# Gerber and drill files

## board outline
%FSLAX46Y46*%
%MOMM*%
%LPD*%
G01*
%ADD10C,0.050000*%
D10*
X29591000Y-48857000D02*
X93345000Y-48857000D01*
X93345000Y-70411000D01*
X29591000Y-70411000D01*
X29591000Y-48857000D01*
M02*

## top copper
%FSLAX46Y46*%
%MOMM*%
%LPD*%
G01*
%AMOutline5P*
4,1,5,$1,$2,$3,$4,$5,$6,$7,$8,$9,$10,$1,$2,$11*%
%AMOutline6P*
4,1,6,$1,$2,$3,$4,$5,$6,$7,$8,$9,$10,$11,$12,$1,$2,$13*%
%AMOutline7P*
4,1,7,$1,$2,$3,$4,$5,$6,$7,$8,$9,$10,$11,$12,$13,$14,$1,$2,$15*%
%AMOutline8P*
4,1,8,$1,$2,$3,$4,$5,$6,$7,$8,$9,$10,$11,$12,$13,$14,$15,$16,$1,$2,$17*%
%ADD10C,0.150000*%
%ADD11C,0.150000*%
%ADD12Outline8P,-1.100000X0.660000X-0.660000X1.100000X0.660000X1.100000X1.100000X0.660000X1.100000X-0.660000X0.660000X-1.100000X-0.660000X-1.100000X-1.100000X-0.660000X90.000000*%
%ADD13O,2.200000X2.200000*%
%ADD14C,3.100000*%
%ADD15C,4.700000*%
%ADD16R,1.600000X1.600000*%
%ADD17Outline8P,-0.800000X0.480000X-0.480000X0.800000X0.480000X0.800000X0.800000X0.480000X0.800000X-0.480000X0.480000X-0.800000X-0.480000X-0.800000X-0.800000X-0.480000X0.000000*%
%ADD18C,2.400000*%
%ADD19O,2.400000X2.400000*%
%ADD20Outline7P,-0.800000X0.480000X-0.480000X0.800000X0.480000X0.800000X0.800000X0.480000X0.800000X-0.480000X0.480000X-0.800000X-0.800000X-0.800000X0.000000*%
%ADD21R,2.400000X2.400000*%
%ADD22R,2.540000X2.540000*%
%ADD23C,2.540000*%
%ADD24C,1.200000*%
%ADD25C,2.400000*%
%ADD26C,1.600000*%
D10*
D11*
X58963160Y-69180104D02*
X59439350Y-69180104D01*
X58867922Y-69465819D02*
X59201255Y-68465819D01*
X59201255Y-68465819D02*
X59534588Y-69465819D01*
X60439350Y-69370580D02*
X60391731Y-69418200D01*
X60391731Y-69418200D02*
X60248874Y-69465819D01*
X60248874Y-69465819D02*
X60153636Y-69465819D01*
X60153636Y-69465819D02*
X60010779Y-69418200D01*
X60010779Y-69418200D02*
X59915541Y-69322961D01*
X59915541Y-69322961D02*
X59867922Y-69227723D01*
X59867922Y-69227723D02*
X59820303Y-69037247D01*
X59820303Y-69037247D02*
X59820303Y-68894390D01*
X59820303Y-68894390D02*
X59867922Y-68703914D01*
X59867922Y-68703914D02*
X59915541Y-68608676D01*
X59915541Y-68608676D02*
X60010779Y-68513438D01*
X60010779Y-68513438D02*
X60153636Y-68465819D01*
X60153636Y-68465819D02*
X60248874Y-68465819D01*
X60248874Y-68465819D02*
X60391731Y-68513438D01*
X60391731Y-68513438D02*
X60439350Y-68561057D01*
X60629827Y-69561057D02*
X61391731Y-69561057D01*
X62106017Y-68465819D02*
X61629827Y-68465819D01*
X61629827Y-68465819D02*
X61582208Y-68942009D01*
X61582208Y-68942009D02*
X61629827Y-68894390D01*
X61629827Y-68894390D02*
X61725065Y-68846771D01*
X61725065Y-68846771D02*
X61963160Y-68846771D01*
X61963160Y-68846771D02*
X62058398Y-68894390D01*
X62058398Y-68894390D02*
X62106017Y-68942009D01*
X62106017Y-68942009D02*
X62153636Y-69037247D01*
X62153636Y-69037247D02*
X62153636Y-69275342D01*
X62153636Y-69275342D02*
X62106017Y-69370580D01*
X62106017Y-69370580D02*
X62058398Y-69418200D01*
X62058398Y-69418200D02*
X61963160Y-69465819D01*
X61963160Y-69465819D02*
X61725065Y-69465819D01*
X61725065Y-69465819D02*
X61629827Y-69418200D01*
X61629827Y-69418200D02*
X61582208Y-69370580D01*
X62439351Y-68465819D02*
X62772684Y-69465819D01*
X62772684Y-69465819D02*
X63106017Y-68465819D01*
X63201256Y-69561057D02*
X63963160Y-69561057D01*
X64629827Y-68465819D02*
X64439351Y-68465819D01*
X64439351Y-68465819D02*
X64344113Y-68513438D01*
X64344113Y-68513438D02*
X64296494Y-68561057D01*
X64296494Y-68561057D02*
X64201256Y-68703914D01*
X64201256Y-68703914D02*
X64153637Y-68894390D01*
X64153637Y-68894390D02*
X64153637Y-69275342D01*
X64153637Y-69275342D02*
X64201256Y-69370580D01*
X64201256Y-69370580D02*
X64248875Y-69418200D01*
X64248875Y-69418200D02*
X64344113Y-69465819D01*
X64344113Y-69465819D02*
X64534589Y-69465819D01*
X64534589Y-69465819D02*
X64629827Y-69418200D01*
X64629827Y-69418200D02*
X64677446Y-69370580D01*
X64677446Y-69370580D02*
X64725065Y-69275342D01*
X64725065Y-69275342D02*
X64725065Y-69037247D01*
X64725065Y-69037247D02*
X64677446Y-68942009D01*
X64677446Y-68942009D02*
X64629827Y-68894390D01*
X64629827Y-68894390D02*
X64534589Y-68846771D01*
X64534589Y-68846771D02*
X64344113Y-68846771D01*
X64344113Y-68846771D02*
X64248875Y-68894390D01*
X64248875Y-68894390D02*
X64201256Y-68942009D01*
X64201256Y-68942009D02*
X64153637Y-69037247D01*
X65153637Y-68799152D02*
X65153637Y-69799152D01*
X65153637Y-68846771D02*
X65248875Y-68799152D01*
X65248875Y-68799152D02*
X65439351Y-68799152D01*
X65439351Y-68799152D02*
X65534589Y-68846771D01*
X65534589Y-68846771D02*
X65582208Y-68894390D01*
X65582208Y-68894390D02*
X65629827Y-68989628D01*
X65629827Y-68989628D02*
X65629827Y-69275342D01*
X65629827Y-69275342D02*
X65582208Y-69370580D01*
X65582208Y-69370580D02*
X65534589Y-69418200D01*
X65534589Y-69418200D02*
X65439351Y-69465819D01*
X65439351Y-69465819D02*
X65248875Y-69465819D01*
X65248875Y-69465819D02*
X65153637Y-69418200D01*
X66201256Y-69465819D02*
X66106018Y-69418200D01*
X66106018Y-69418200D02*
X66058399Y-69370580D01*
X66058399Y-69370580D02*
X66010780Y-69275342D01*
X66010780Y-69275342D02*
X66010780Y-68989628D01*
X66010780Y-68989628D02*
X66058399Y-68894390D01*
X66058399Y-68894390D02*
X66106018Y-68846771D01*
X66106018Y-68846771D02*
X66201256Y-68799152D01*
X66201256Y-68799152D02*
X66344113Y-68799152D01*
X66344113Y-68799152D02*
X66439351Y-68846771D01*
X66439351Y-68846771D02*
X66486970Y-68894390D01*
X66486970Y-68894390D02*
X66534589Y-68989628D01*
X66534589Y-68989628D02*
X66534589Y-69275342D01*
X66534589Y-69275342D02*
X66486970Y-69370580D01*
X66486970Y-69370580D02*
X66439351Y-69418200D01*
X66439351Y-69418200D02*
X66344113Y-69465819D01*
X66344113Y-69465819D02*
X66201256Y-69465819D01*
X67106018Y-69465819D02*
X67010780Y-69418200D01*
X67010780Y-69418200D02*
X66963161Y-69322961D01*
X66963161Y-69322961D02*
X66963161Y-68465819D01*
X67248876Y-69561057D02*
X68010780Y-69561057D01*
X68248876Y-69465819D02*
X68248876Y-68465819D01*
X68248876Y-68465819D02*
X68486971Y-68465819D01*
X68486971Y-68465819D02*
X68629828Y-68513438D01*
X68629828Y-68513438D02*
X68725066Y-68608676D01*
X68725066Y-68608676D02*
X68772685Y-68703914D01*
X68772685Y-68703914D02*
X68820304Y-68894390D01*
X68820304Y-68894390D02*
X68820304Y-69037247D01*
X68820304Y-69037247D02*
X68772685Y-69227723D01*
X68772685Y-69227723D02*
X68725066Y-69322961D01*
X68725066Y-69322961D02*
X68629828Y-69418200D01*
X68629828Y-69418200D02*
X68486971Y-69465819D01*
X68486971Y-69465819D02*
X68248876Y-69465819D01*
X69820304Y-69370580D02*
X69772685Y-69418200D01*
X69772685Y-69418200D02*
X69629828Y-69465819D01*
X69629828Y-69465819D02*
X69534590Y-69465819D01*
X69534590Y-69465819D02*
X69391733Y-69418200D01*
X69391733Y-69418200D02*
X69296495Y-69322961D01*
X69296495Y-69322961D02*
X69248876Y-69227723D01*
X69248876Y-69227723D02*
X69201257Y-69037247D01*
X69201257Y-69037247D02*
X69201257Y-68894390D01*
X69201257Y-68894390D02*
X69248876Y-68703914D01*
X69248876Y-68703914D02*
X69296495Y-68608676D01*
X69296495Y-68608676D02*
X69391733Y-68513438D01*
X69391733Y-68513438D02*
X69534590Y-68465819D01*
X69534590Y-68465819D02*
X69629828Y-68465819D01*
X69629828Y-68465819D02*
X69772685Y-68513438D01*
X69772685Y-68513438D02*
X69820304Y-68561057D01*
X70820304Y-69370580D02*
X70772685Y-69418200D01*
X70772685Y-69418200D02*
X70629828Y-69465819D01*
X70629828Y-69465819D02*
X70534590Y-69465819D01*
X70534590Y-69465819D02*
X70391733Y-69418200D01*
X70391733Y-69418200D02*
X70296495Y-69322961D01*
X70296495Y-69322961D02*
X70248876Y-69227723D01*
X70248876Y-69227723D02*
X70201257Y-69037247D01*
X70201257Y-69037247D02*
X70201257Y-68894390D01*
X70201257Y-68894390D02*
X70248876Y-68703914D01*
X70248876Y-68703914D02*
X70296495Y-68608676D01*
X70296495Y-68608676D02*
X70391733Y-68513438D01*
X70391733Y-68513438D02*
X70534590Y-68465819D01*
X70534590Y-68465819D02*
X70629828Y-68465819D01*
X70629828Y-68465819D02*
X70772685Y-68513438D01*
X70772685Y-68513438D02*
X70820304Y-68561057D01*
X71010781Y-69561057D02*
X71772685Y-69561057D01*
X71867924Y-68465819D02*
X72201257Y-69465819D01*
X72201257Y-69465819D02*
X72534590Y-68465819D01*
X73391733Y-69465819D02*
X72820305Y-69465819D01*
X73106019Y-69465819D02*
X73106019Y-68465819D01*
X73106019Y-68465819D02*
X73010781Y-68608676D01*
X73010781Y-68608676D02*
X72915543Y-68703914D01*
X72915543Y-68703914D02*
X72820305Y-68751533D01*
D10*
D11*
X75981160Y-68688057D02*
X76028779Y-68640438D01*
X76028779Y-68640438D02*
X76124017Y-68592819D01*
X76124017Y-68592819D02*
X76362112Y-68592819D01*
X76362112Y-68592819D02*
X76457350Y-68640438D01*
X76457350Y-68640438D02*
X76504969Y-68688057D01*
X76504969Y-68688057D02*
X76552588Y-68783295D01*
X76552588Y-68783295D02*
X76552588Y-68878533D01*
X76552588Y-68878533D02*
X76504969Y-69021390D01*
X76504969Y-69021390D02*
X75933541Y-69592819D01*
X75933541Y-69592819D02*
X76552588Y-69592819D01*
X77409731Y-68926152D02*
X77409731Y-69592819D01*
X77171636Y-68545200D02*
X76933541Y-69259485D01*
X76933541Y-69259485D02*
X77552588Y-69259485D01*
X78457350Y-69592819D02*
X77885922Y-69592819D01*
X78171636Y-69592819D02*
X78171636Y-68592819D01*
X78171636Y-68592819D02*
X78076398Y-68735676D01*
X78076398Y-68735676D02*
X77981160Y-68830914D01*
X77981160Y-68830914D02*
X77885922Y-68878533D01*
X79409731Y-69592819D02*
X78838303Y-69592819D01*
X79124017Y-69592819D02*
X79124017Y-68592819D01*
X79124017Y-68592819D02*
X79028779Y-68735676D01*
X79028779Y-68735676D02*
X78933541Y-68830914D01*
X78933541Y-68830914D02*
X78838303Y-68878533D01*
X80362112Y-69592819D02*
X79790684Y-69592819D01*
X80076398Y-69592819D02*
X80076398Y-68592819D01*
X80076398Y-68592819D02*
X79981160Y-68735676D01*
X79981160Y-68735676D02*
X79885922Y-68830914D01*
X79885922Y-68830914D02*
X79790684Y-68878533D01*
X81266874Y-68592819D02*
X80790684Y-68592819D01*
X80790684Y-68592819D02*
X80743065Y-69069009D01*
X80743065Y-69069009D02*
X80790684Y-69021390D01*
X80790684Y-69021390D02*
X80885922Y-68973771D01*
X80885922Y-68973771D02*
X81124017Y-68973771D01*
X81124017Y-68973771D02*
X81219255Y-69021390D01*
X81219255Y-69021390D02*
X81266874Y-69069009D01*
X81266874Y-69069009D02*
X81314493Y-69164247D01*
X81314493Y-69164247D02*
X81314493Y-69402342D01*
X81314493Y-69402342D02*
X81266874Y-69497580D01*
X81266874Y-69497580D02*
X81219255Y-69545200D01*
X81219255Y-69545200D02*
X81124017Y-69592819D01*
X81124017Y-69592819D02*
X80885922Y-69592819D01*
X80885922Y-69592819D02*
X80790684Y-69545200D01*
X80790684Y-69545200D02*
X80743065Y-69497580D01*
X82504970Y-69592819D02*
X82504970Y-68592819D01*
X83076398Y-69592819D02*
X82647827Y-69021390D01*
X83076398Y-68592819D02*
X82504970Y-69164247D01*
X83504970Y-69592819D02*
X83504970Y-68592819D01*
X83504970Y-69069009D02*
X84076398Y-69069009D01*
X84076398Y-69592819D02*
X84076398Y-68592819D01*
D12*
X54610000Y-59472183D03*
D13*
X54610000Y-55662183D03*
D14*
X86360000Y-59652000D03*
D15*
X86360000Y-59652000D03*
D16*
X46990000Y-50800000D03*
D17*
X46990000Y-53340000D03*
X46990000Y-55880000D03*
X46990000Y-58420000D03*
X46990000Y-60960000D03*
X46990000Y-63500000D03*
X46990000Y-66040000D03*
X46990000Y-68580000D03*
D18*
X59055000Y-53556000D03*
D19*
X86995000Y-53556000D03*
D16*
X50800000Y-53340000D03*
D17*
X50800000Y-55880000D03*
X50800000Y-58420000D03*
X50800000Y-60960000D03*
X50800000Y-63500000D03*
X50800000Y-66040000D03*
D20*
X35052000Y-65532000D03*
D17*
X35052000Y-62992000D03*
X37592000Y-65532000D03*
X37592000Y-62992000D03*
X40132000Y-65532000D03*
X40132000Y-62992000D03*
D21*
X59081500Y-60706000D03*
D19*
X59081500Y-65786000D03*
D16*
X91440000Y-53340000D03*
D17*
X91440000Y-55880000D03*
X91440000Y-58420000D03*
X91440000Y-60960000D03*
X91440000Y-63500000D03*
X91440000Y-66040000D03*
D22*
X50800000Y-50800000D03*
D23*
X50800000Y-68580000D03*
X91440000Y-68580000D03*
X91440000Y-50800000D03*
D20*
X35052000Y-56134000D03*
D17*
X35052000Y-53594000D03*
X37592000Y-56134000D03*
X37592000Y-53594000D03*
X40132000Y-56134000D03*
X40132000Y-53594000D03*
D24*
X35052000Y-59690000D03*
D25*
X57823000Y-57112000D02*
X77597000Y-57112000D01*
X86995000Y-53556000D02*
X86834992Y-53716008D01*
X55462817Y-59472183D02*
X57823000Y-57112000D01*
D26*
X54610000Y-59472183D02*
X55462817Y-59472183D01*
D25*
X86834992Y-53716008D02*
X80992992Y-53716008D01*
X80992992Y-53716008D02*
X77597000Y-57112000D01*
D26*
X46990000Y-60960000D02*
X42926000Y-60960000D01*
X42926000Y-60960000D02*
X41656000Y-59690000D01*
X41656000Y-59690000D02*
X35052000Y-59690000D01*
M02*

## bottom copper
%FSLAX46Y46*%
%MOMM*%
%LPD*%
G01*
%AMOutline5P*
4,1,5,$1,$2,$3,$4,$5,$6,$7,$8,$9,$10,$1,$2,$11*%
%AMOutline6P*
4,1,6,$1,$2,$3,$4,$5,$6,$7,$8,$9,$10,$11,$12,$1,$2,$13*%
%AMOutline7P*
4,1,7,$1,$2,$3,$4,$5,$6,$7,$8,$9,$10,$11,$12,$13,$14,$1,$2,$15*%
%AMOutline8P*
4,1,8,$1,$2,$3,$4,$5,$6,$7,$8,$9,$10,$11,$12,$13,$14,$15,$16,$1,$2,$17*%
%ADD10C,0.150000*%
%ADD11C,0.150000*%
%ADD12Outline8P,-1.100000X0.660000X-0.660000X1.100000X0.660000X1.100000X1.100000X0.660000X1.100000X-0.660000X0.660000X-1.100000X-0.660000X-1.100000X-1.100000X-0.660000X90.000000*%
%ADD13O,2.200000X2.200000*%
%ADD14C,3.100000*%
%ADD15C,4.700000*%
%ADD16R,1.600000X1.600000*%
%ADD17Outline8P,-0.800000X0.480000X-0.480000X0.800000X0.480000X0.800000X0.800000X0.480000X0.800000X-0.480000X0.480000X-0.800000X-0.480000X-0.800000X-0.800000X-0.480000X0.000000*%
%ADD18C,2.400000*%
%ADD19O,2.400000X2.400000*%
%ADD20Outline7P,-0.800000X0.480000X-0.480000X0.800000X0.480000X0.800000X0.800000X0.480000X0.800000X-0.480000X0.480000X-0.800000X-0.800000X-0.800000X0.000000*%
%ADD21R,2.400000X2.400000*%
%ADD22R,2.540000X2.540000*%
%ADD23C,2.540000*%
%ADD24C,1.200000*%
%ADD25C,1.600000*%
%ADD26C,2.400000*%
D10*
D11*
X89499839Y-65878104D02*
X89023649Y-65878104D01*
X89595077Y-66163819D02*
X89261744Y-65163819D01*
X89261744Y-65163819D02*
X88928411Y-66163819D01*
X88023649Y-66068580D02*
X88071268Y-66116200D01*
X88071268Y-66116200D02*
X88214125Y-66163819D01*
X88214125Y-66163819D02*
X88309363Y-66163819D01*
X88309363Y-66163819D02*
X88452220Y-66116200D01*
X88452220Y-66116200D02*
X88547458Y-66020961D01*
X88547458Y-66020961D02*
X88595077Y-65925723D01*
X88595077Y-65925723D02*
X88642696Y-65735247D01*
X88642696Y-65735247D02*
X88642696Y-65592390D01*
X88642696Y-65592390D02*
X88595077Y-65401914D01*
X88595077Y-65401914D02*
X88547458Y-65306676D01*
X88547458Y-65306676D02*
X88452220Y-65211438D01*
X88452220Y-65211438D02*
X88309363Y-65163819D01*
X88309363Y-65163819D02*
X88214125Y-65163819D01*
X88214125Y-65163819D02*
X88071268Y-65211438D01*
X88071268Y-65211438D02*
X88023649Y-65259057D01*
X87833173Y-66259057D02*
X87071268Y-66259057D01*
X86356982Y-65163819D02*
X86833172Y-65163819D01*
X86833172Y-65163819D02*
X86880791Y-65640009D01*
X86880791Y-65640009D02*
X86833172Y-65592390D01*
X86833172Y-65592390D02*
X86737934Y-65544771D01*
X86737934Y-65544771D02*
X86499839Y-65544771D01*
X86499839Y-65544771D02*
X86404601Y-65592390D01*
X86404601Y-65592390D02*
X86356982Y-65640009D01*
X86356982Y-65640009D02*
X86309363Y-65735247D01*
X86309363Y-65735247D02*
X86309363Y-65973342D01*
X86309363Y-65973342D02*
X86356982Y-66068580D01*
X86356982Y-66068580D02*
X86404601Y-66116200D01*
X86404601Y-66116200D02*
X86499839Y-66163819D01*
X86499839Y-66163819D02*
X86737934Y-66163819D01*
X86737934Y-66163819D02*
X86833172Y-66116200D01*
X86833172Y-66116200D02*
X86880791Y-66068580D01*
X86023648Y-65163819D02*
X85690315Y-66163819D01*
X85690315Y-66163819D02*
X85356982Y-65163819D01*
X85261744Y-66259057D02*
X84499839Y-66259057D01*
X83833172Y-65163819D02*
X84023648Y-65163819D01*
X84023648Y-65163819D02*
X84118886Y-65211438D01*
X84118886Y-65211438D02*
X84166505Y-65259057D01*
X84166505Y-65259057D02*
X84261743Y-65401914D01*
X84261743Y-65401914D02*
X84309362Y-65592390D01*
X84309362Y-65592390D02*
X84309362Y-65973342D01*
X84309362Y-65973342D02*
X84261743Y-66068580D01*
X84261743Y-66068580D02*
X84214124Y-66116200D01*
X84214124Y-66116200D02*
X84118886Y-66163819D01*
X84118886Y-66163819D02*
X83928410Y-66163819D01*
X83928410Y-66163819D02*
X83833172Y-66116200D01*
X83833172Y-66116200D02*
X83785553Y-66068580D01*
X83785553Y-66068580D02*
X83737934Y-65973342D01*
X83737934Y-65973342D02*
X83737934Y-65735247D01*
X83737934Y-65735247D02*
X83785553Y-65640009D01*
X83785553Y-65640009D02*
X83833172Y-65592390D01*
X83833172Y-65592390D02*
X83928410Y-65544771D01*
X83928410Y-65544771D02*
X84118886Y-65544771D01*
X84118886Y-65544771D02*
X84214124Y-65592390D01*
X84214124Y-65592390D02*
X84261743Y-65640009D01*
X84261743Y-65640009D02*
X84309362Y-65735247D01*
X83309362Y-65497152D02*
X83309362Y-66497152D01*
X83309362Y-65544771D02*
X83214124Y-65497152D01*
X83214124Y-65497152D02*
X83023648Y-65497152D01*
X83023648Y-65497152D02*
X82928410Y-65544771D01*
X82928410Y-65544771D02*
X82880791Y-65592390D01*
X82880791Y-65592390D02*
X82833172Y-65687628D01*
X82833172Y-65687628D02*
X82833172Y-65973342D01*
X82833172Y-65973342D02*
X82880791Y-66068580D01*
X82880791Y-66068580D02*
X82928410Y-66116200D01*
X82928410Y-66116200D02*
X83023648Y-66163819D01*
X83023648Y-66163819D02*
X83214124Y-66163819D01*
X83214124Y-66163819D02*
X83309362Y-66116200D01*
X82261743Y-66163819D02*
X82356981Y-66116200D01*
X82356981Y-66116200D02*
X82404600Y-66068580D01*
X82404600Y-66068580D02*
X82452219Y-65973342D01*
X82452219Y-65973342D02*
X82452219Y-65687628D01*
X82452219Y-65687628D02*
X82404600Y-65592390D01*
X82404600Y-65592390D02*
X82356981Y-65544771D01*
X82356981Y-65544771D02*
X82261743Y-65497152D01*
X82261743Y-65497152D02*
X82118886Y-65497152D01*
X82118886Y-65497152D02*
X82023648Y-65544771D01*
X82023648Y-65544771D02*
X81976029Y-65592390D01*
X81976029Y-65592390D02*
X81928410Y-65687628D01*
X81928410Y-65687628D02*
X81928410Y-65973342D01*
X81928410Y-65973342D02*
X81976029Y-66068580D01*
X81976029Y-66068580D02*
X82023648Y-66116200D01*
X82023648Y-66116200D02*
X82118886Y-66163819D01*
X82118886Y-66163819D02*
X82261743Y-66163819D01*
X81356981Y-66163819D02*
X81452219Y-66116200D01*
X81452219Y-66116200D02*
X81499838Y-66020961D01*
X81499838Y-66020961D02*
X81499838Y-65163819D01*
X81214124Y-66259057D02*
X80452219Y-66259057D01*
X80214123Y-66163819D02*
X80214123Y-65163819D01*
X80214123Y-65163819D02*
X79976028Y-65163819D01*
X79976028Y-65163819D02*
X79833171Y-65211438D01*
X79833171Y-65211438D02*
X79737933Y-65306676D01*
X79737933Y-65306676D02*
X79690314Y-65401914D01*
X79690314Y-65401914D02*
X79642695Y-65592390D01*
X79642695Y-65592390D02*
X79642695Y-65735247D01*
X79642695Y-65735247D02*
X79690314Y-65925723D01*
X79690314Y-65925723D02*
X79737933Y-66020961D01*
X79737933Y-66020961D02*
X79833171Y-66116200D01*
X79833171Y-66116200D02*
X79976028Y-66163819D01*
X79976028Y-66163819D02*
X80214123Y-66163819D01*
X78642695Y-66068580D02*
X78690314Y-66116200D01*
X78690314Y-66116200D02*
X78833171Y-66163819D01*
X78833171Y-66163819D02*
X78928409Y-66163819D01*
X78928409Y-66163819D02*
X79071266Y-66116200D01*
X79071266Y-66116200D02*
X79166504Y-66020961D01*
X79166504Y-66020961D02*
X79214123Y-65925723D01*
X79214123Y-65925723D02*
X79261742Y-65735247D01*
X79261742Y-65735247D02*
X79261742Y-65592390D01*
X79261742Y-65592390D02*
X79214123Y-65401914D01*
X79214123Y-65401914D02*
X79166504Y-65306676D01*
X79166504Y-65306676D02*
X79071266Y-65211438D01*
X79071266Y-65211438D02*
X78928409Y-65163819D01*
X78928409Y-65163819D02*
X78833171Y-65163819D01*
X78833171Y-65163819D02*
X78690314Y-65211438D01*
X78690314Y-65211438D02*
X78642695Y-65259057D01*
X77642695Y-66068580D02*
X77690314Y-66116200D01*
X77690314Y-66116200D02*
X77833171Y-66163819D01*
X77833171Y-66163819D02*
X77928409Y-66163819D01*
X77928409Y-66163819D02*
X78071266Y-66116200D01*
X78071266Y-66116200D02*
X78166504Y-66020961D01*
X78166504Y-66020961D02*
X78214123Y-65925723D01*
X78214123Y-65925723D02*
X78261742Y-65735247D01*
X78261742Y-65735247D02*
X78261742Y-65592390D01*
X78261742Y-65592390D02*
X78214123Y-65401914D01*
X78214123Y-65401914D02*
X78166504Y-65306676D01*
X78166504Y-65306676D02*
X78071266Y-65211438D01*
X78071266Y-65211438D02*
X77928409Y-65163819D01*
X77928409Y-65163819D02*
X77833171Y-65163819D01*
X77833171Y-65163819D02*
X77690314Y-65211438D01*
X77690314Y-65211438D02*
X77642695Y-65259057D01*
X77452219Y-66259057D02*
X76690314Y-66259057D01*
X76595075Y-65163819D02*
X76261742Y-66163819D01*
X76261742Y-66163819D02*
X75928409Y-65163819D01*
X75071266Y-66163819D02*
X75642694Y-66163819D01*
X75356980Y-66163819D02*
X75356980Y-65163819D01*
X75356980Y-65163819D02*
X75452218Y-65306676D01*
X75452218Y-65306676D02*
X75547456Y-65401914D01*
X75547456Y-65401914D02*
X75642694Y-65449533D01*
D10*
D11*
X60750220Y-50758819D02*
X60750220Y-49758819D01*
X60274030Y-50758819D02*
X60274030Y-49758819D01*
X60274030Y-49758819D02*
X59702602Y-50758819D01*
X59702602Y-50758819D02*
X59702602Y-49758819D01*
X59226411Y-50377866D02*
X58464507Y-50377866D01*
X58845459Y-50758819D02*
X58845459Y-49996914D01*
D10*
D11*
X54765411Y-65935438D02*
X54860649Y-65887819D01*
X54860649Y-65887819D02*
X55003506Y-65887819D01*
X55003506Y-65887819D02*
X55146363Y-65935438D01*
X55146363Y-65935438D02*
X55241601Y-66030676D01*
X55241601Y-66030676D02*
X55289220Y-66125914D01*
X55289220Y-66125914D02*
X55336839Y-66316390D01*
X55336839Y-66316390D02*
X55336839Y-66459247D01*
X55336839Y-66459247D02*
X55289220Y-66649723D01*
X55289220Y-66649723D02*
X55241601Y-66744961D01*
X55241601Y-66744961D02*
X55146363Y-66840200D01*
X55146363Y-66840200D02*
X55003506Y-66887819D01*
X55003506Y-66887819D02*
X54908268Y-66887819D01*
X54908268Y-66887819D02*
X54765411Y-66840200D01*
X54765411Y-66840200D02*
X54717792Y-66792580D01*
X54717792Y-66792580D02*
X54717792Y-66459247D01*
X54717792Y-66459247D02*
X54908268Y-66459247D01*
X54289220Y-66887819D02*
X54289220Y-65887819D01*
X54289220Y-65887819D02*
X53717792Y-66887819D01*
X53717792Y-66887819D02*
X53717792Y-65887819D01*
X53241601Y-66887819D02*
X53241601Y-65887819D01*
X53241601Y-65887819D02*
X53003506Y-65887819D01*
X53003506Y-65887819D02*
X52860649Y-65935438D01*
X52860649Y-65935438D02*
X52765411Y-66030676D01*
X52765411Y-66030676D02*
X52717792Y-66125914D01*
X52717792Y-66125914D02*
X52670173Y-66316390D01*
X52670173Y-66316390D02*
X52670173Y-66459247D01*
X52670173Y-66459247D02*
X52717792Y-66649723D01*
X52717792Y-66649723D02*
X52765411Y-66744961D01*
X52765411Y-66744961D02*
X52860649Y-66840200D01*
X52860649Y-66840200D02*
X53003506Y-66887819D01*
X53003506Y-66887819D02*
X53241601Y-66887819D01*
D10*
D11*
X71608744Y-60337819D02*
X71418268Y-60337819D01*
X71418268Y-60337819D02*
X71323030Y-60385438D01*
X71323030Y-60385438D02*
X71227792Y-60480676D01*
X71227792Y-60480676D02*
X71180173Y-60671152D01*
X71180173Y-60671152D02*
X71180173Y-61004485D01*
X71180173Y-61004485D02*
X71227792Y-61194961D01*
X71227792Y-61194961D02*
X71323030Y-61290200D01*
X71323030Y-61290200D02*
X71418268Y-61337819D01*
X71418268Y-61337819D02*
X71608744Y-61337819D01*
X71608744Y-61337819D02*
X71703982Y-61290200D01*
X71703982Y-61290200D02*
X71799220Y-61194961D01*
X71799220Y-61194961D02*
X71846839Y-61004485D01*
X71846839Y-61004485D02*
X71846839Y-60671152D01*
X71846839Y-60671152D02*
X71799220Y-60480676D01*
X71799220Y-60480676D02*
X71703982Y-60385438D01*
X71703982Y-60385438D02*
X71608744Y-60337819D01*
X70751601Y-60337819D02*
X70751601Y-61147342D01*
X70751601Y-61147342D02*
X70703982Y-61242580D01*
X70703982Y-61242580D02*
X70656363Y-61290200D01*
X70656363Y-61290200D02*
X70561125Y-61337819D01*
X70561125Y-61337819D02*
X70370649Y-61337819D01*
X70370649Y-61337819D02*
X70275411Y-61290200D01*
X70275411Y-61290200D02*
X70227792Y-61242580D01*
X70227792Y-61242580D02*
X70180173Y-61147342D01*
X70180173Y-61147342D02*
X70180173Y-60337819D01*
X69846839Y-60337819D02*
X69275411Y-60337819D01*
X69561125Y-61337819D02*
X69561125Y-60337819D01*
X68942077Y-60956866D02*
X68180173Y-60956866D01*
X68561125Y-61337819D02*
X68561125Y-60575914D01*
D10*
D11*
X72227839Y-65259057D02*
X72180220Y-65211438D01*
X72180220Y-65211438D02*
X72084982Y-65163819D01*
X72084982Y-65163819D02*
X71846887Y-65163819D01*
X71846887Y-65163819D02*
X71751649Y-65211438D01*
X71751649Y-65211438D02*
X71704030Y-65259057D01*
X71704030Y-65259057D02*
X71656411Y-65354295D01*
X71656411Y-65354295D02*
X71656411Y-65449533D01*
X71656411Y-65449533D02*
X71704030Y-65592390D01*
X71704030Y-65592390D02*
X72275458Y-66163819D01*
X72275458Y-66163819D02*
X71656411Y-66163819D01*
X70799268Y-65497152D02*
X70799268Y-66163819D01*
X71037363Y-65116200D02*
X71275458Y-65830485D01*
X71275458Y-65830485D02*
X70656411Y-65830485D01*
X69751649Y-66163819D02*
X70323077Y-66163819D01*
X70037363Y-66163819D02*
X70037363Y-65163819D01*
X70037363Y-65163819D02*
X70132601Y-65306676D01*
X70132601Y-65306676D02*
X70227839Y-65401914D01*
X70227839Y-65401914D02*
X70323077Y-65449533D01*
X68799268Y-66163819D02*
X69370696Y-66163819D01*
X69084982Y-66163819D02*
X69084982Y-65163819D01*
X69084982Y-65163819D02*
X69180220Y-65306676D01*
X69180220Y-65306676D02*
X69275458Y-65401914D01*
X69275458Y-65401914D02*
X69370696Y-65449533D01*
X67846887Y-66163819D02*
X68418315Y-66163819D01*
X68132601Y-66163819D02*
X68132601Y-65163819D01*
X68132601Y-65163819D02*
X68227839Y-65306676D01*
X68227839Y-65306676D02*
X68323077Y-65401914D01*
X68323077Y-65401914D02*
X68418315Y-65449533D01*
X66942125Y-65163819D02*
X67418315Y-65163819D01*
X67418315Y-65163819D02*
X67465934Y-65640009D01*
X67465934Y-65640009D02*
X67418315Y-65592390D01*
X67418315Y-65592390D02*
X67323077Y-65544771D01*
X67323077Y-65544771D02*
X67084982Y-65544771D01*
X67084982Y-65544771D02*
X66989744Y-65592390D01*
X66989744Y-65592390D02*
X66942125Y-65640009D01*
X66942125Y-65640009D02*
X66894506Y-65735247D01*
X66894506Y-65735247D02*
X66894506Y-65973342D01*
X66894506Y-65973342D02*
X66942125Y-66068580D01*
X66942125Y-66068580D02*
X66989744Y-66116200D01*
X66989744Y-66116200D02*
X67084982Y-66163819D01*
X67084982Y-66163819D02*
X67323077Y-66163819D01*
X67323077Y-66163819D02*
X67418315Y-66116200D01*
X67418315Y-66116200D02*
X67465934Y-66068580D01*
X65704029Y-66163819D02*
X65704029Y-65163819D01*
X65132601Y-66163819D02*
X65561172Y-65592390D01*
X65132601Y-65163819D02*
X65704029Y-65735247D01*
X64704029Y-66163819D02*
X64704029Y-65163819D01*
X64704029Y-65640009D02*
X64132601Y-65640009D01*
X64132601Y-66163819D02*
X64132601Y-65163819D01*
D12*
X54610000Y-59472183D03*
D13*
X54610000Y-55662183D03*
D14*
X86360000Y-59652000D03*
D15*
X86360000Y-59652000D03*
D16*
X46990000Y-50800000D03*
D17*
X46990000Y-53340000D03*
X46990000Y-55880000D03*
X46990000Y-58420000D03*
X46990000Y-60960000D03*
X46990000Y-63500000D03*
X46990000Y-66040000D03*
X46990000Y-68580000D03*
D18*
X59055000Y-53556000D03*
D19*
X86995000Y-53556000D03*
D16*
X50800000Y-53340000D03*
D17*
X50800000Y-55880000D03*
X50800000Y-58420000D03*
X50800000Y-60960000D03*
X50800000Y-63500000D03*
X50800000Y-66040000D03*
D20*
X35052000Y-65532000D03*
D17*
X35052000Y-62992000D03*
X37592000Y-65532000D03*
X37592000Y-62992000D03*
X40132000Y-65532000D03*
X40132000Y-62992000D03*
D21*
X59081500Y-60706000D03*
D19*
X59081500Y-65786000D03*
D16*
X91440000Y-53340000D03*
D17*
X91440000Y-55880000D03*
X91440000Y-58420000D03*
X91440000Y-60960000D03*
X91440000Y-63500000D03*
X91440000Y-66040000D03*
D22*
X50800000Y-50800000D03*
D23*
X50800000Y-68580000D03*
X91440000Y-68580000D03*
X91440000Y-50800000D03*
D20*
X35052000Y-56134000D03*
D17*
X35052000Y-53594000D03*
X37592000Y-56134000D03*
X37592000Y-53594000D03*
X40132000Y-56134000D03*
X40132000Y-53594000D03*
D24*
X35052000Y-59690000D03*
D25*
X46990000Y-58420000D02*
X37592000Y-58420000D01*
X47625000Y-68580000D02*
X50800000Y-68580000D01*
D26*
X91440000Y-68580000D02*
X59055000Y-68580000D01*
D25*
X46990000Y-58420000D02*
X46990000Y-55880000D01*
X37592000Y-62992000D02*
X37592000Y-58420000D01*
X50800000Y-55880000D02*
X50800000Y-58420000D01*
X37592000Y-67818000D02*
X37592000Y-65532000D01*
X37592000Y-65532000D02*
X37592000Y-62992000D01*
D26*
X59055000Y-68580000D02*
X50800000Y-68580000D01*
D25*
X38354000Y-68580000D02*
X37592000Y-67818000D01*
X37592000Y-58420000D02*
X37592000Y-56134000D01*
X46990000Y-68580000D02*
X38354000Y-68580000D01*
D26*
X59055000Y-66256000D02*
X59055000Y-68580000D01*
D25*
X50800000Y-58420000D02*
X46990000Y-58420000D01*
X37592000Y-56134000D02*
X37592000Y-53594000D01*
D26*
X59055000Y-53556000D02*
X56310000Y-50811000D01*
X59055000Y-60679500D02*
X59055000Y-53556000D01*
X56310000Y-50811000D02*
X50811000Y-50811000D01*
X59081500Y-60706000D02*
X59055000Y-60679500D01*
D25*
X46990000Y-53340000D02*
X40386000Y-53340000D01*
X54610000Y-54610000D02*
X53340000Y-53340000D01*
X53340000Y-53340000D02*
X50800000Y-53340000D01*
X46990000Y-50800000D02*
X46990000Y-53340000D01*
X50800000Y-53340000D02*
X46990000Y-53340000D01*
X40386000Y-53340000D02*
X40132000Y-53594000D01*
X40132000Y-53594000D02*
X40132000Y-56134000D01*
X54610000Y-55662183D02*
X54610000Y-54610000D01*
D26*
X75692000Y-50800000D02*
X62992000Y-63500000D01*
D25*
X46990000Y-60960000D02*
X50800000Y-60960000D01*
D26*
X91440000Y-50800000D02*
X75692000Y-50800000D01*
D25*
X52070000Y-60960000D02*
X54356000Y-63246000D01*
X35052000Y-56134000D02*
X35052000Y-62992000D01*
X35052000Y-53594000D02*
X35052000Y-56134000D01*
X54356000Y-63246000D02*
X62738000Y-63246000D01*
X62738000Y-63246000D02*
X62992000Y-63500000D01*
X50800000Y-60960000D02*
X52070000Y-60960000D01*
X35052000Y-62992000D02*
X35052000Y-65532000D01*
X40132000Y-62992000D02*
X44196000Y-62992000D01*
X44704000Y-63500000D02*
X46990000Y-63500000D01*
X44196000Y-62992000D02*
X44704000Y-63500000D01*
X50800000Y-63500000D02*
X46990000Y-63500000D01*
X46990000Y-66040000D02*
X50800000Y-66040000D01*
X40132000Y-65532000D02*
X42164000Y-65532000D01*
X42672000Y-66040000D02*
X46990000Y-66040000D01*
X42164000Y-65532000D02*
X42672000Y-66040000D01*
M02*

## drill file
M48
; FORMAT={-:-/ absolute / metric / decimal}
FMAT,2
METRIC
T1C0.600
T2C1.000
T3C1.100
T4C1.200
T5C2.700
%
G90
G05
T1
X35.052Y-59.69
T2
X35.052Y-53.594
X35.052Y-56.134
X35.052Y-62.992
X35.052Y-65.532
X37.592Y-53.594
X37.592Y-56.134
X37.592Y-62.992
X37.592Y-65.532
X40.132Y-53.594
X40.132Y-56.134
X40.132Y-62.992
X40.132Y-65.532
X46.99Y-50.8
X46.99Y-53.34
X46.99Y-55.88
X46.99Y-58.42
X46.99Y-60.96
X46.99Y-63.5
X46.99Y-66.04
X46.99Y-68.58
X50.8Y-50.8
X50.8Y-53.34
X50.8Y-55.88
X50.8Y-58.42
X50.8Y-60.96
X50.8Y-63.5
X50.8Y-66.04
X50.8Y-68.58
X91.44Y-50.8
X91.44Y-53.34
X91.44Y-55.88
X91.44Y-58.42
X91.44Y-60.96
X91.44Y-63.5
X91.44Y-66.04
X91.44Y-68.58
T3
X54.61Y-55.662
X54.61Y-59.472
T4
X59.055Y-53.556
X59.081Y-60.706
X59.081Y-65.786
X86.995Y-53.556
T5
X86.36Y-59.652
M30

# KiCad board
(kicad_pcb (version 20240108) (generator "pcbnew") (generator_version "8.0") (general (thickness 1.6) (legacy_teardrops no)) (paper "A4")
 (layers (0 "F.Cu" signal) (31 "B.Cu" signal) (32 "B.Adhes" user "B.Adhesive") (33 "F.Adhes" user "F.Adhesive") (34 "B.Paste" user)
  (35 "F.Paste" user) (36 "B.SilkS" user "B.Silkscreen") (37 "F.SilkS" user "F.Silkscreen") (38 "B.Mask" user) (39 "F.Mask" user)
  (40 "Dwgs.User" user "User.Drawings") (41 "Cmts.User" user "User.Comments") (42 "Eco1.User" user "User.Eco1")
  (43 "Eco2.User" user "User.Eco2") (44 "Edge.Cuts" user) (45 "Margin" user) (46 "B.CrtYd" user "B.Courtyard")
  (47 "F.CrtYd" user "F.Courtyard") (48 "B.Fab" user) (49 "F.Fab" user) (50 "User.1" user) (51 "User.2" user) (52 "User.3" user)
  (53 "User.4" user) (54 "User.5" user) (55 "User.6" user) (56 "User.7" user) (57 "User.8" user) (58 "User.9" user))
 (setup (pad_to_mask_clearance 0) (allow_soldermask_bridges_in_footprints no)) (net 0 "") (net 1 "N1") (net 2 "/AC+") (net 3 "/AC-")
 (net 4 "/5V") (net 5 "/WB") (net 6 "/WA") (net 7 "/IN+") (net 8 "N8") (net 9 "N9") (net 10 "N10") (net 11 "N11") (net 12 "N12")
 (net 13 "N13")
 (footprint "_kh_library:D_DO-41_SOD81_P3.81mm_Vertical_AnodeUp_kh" (layer "F.Cu") (at 54.61 59.472183 90)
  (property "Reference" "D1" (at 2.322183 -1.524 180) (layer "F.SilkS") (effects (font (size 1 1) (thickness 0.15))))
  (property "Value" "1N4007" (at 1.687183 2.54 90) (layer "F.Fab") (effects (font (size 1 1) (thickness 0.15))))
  (pad "1" thru_hole roundrect (at 0 0 90) (size 2.2 2.2) (drill 1.1) (layers "*.Cu" "*.Mask") (remove_unused_layers no)
   (roundrect_rratio 0) (chamfer_ratio 0.2) (chamfer top_left top_right bottom_left bottom_right) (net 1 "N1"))
  (pad "2" thru_hole oval (at 3.81 0 90) (size 2.2 2.2) (drill 1.1) (layers "*.Cu" "*.Mask") (remove_unused_layers no) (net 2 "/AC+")))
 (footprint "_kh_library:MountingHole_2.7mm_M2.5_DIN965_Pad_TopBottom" (layer "F.Cu") (at 86.36 59.652)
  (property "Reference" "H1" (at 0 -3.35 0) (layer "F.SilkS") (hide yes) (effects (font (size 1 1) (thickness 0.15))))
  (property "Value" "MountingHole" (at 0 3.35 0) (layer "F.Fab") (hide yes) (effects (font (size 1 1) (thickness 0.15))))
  (pad "1" thru_hole circle (at 0 0) (size 3.1 3.1) (drill 2.7) (layers "*.Cu" "*.Mask") (remove_unused_layers no))
  (pad "1" connect circle (at 0 0) (size 4.7 4.7) (layers "F.Cu" "F.Mask"))
  (pad "1" connect circle (at 0 0) (size 4.7 4.7) (layers "B.Cu" "B.Mask")))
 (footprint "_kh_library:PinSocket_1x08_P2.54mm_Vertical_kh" (layer "F.Cu") (at 46.99 50.8)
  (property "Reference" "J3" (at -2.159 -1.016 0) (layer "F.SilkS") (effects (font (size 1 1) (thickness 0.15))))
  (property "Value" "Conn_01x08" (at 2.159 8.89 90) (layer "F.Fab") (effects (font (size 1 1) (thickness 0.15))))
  (pad "1" thru_hole rect (at 0 0) (size 1.6 1.6) (drill 1) (layers "*.Cu" "*.Mask") (remove_unused_layers no) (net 2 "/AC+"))
  (pad "2" thru_hole roundrect (at 0 2.54) (size 1.6 1.6) (drill 1) (layers "*.Cu" "*.Mask") (remove_unused_layers no) (roundrect_rratio 0)
   (chamfer_ratio 0.2) (chamfer top_left top_right bottom_left bottom_right) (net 2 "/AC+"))
  (pad "3" thru_hole roundrect (at 0 5.08) (size 1.6 1.6) (drill 1) (layers "*.Cu" "*.Mask") (remove_unused_layers no) (roundrect_rratio 0)
   (chamfer_ratio 0.2) (chamfer top_left top_right bottom_left bottom_right) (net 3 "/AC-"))
  (pad "4" thru_hole roundrect (at 0 7.62) (size 1.6 1.6) (drill 1) (layers "*.Cu" "*.Mask") (remove_unused_layers no) (roundrect_rratio 0)
   (chamfer_ratio 0.2) (chamfer top_left top_right bottom_left bottom_right) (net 3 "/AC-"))
  (pad "5" thru_hole roundrect (at 0 10.16) (size 1.6 1.6) (drill 1) (layers "*.Cu" "*.Mask") (remove_unused_layers no) (roundrect_rratio 0)
   (chamfer_ratio 0.2) (chamfer top_left top_right bottom_left bottom_right) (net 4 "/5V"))
  (pad "6" thru_hole roundrect (at 0 12.7) (size 1.6 1.6) (drill 1) (layers "*.Cu" "*.Mask") (remove_unused_layers no) (roundrect_rratio 0)
   (chamfer_ratio 0.2) (chamfer top_left top_right bottom_left bottom_right) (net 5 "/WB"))
  (pad "7" thru_hole roundrect (at 0 15.24) (size 1.6 1.6) (drill 1) (layers "*.Cu" "*.Mask") (remove_unused_layers no) (roundrect_rratio 0)
   (chamfer_ratio 0.2) (chamfer top_left top_right bottom_left bottom_right) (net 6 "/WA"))
  (pad "8" thru_hole roundrect (at 0 17.78) (size 1.6 1.6) (drill 1) (layers "*.Cu" "*.Mask") (remove_unused_layers no) (roundrect_rratio 0)
   (chamfer_ratio 0.2) (chamfer top_left top_right bottom_left bottom_right) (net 3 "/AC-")))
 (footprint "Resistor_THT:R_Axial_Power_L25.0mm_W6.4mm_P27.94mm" (layer "F.Cu") (at 59.055 53.556)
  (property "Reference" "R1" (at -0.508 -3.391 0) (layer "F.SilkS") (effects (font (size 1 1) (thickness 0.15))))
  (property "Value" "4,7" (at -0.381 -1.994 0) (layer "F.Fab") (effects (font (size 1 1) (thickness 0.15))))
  (pad "1" thru_hole circle (at 0 0) (size 2.4 2.4) (drill 1.2) (layers "*.Cu" "*.Mask") (remove_unused_layers no) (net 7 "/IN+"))
  (pad "2" thru_hole oval (at 27.94 0) (size 2.4 2.4) (drill 1.2) (layers "*.Cu" "*.Mask") (remove_unused_layers no) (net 1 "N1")))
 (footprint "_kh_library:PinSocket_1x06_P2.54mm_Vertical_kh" (layer "F.Cu") (at 50.8 53.34)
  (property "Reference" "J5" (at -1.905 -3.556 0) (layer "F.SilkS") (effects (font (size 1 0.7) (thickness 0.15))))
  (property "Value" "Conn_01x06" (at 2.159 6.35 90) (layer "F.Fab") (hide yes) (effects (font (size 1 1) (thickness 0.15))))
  (pad "1" thru_hole rect (at 0 0) (size 1.6 1.6) (drill 1) (layers "*.Cu" "*.Mask") (remove_unused_layers no) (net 2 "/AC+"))
  (pad "2" thru_hole roundrect (at 0 2.54) (size 1.6 1.6) (drill 1) (layers "*.Cu" "*.Mask") (remove_unused_layers no) (roundrect_rratio 0)
   (chamfer_ratio 0.2) (chamfer top_left top_right bottom_left bottom_right) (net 3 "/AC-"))
  (pad "3" thru_hole roundrect (at 0 5.08) (size 1.6 1.6) (drill 1) (layers "*.Cu" "*.Mask") (remove_unused_layers no) (roundrect_rratio 0)
   (chamfer_ratio 0.2) (chamfer top_left top_right bottom_left bottom_right) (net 3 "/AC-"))
  (pad "4" thru_hole roundrect (at 0 7.62) (size 1.6 1.6) (drill 1) (layers "*.Cu" "*.Mask") (remove_unused_layers no) (roundrect_rratio 0)
   (chamfer_ratio 0.2) (chamfer top_left top_right bottom_left bottom_right) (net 4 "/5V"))
  (pad "5" thru_hole roundrect (at 0 10.16) (size 1.6 1.6) (drill 1) (layers "*.Cu" "*.Mask") (remove_unused_layers no) (roundrect_rratio 0)
   (chamfer_ratio 0.2) (chamfer top_left top_right bottom_left bottom_right) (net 5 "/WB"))
  (pad "6" thru_hole roundrect (at 0 12.7) (size 1.6 1.6) (drill 1) (layers "*.Cu" "*.Mask") (remove_unused_layers no) (roundrect_rratio 0)
   (chamfer_ratio 0.2) (chamfer top_left top_right bottom_left bottom_right) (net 6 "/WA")))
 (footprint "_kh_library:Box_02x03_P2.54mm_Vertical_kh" (layer "F.Cu") (at 35.052 65.532)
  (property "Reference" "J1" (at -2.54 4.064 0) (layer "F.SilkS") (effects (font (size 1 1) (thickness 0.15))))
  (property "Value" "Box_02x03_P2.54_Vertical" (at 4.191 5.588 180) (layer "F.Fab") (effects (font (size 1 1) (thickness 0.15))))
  (pad "1" thru_hole roundrect (at 0 0) (size 1.6 1.6) (drill 1) (layers "*.Cu" "*.Mask") (remove_unused_layers no) (roundrect_rratio 0)
   (chamfer_ratio 0.2) (chamfer top_left top_right bottom_right) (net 4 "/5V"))
  (pad "2" thru_hole roundrect (at 0 -2.54) (size 1.6 1.6) (drill 1) (layers "*.Cu" "*.Mask") (remove_unused_layers no) (roundrect_rratio 0)
   (chamfer_ratio 0.2) (chamfer top_left top_right bottom_left bottom_right) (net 4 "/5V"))
  (pad "3" thru_hole roundrect (at 2.54 0) (size 1.6 1.6) (drill 1) (layers "*.Cu" "*.Mask") (remove_unused_layers no) (roundrect_rratio 0)
   (chamfer_ratio 0.2) (chamfer top_left top_right bottom_left bottom_right) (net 3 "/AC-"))
  (pad "4" thru_hole roundrect (at 2.54 -2.54) (size 1.6 1.6) (drill 1) (layers "*.Cu" "*.Mask") (remove_unused_layers no)
   (roundrect_rratio 0) (chamfer_ratio 0.2) (chamfer top_left top_right bottom_left bottom_right) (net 3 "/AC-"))
  (pad "5" thru_hole roundrect (at 5.08 0) (size 1.6 1.6) (drill 1) (layers "*.Cu" "*.Mask") (remove_unused_layers no) (roundrect_rratio 0)
   (chamfer_ratio 0.2) (chamfer top_left top_right bottom_left bottom_right) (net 6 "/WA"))
  (pad "6" thru_hole roundrect (at 5.08 -2.54) (size 1.6 1.6) (drill 1) (layers "*.Cu" "*.Mask") (remove_unused_layers no)
   (roundrect_rratio 0) (chamfer_ratio 0.2) (chamfer top_left top_right bottom_left bottom_right) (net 5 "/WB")))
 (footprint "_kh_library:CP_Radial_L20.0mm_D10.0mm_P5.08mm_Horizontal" (layer "F.Cu") (at 59.0815 63.246)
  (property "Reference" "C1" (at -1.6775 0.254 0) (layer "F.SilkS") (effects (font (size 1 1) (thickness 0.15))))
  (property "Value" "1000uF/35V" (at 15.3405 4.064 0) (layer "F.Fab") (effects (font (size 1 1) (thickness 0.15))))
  (pad "1" thru_hole rect (at 0 -2.54) (size 2.4 2.4) (drill 1.2) (layers "*.Cu" "*.Mask") (remove_unused_layers no) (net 7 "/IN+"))
  (pad "2" thru_hole oval (at 0 2.54) (size 2.4 2.4) (drill 1.2) (layers "*.Cu" "*.Mask") (remove_unused_layers no) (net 3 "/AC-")))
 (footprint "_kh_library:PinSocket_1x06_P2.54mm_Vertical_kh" (layer "F.Cu") (at 91.44 53.34)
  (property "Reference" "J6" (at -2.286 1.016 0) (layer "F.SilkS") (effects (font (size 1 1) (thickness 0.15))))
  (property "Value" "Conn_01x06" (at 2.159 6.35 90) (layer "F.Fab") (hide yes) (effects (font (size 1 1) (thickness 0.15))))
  (pad "1" thru_hole rect (at 0 0) (size 1.6 1.6) (drill 1) (layers "*.Cu" "*.Mask") (remove_unused_layers no) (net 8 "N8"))
  (pad "2" thru_hole roundrect (at 0 2.54) (size 1.6 1.6) (drill 1) (layers "*.Cu" "*.Mask") (remove_unused_layers no) (roundrect_rratio 0)
   (chamfer_ratio 0.2) (chamfer top_left top_right bottom_left bottom_right) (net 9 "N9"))
  (pad "3" thru_hole roundrect (at 0 5.08) (size 1.6 1.6) (drill 1) (layers "*.Cu" "*.Mask") (remove_unused_layers no) (roundrect_rratio 0)
   (chamfer_ratio 0.2) (chamfer top_left top_right bottom_left bottom_right) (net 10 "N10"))
  (pad "4" thru_hole roundrect (at 0 7.62) (size 1.6 1.6) (drill 1) (layers "*.Cu" "*.Mask") (remove_unused_layers no) (roundrect_rratio 0)
   (chamfer_ratio 0.2) (chamfer top_left top_right bottom_left bottom_right) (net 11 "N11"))
  (pad "5" thru_hole roundrect (at 0 10.16) (size 1.6 1.6) (drill 1) (layers "*.Cu" "*.Mask") (remove_unused_layers no) (roundrect_rratio 0)
   (chamfer_ratio 0.2) (chamfer top_left top_right bottom_left bottom_right) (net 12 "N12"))
  (pad "6" thru_hole roundrect (at 0 12.7) (size 1.6 1.6) (drill 1) (layers "*.Cu" "*.Mask") (remove_unused_layers no) (roundrect_rratio 0)
   (chamfer_ratio 0.2) (chamfer top_left top_right bottom_left bottom_right) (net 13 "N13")))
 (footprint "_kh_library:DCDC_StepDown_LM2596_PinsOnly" (layer "F.Cu") (at 50.8 50.8)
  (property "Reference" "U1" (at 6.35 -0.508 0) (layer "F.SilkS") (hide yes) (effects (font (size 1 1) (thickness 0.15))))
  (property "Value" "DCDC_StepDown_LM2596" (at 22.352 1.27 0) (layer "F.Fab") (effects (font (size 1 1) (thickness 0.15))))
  (pad "1" thru_hole rect (at 0 0) (size 2.54 2.54) (drill 1) (layers "*.Cu" "*.Mask") (remove_unused_layers no) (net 7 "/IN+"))
  (pad "2" thru_hole circle (at 0 17.78) (size 2.54 2.54) (drill 1) (layers "*.Cu" "*.Mask") (remove_unused_layers no) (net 3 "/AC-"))
  (pad "3" thru_hole circle (at 40.64 17.78) (size 2.54 2.54) (drill 1) (layers "*.Cu" "*.Mask") (remove_unused_layers no) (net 3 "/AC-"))
  (pad "4" thru_hole circle (at 40.64 0) (size 2.54 2.54) (drill 1) (layers "*.Cu" "*.Mask") (remove_unused_layers no) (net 4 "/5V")))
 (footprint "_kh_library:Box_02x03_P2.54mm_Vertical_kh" (layer "F.Cu") (at 35.052 56.134)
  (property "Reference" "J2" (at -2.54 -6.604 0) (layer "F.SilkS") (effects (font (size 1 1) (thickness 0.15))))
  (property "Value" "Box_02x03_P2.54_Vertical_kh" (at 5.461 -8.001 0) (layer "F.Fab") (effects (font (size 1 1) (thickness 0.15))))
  (pad "1" thru_hole roundrect (at 0 0) (size 1.6 1.6) (drill 1) (layers "*.Cu" "*.Mask") (remove_unused_layers no) (roundrect_rratio 0)
   (chamfer_ratio 0.2) (chamfer top_left top_right bottom_right) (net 4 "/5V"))
  (pad "2" thru_hole roundrect (at 0 -2.54) (size 1.6 1.6) (drill 1) (layers "*.Cu" "*.Mask") (remove_unused_layers no) (roundrect_rratio 0)
   (chamfer_ratio 0.2) (chamfer top_left top_right bottom_left bottom_right) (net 4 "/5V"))
  (pad "3" thru_hole roundrect (at 2.54 0) (size 1.6 1.6) (drill 1) (layers "*.Cu" "*.Mask") (remove_unused_layers no) (roundrect_rratio 0)
   (chamfer_ratio 0.2) (chamfer top_left top_right bottom_left bottom_right) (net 3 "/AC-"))
  (pad "4" thru_hole roundrect (at 2.54 -2.54) (size 1.6 1.6) (drill 1) (layers "*.Cu" "*.Mask") (remove_unused_layers no)
   (roundrect_rratio 0) (chamfer_ratio 0.2) (chamfer top_left top_right bottom_left bottom_right) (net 3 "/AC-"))
  (pad "5" thru_hole roundrect (at 5.08 0) (size 1.6 1.6) (drill 1) (layers "*.Cu" "*.Mask") (remove_unused_layers no) (roundrect_rratio 0)
   (chamfer_ratio 0.2) (chamfer top_left top_right bottom_left bottom_right) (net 2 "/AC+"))
  (pad "6" thru_hole roundrect (at 5.08 -2.54) (size 1.6 1.6) (drill 1) (layers "*.Cu" "*.Mask") (remove_unused_layers no)
   (roundrect_rratio 0) (chamfer_ratio 0.2) (chamfer top_left top_right bottom_left bottom_right) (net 2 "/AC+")))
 (gr_rect (start 29.591 48.857) (end 93.345 70.411) (stroke (width 0.05) (type default)) (fill none) (layer "Edge.Cuts"))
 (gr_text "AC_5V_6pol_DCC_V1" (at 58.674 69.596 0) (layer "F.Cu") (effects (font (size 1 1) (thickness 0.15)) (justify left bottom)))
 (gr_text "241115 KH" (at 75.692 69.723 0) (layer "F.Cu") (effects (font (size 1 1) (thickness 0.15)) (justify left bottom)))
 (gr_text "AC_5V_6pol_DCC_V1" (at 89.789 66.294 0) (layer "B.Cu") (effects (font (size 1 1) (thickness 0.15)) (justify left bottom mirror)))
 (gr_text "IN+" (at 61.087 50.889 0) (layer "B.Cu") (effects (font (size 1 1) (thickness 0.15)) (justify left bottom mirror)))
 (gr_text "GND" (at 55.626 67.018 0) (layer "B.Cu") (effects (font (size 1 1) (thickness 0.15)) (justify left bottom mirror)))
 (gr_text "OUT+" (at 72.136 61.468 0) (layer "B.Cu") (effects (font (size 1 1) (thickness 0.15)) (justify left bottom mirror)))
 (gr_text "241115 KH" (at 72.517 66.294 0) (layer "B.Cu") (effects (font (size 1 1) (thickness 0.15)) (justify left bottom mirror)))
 (segment (start 46.99 58.42) (end 37.592 58.42) (width 1.6) (layer "B.Cu") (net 3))
 (segment (start 47.625 68.58) (end 50.8 68.58) (width 1.6) (layer "B.Cu") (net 3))
 (segment (start 91.44 68.58) (end 59.055 68.58) (width 2.4) (layer "B.Cu") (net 3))
 (segment (start 46.99 58.42) (end 46.99 55.88) (width 1.6) (layer "B.Cu") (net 3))
 (segment (start 37.592 62.992) (end 37.592 58.42) (width 1.6) (layer "B.Cu") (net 3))
 (segment (start 50.8 55.88) (end 50.8 58.42) (width 1.6) (layer "B.Cu") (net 3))
 (segment (start 37.592 67.818) (end 37.592 65.532) (width 1.6) (layer "B.Cu") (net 3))
 (segment (start 37.592 65.532) (end 37.592 62.992) (width 1.6) (layer "B.Cu") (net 3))
 (segment (start 59.055 68.58) (end 50.8 68.58) (width 2.4) (layer "B.Cu") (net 3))
 (segment (start 38.354 68.58) (end 37.592 67.818) (width 1.6) (layer "B.Cu") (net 3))
 (segment (start 37.592 58.42) (end 37.592 56.134) (width 1.6) (layer "B.Cu") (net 3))
 (segment (start 46.99 68.58) (end 38.354 68.58) (width 1.6) (layer "B.Cu") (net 3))
 (segment (start 59.055 66.256) (end 59.055 68.58) (width 2.4) (layer "B.Cu") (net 3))
 (segment (start 50.8 58.42) (end 46.99 58.42) (width 1.6) (layer "B.Cu") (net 3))
 (segment (start 37.592 56.134) (end 37.592 53.594) (width 1.6) (layer "B.Cu") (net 3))
 (segment (start 59.055 53.556) (end 56.31 50.811) (width 2.4) (layer "B.Cu") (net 7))
 (segment (start 59.055 60.6795) (end 59.055 53.556) (width 2.4) (layer "B.Cu") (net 7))
 (segment (start 56.31 50.811) (end 50.811 50.811) (width 2.4) (layer "B.Cu") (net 7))
 (segment (start 59.0815 60.706) (end 59.055 60.6795) (width 2.4) (layer "B.Cu") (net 7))
 (segment (start 46.99 53.34) (end 40.386 53.34) (width 1.6) (layer "B.Cu") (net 2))
 (segment (start 54.61 54.61) (end 53.34 53.34) (width 1.6) (layer "B.Cu") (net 2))
 (segment (start 53.34 53.34) (end 50.8 53.34) (width 1.6) (layer "B.Cu") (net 2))
 (segment (start 46.99 50.8) (end 46.99 53.34) (width 1.6) (layer "B.Cu") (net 2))
 (segment (start 50.8 53.34) (end 46.99 53.34) (width 1.6) (layer "B.Cu") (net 2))
 (segment (start 40.386 53.34) (end 40.132 53.594) (width 1.6) (layer "B.Cu") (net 2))
 (segment (start 40.132 53.594) (end 40.132 56.134) (width 1.6) (layer "B.Cu") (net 2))
 (segment (start 54.61 55.662183) (end 54.61 54.61) (width 1.6) (layer "B.Cu") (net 2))
 (segment (start 57.823 57.112) (end 77.597 57.112) (width 2.4) (layer "F.Cu") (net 1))
 (segment (start 86.995 53.556) (end 86.834992 53.716008) (width 2.4) (layer "F.Cu") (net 1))
 (segment (start 55.462817 59.472183) (end 57.823 57.112) (width 2.4) (layer "F.Cu") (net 1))
 (segment (start 54.61 59.472183) (end 55.462817 59.472183) (width 1.6) (layer "F.Cu") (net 1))
 (segment (start 86.834992 53.716008) (end 80.992992 53.716008) (width 2.4) (layer "F.Cu") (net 1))
 (segment (start 80.992992 53.716008) (end 77.597 57.112) (width 2.4) (layer "F.Cu") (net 1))
 (segment (start 46.99 60.96) (end 42.926 60.96) (width 1.6) (layer "F.Cu") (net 4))
 (segment (start 42.926 60.96) (end 41.656 59.69) (width 1.6) (layer "F.Cu") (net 4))
 (segment (start 41.656 59.69) (end 35.052 59.69) (width 1.6) (layer "F.Cu") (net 4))
 (via (at 35.052 59.69) (size 1.2) (drill 0.6) (layers "F.Cu" "B.Cu") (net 4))
 (segment (start 75.692 50.8) (end 62.992 63.5) (width 2.4) (layer "B.Cu") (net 4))
 (segment (start 46.99 60.96) (end 50.8 60.96) (width 1.6) (layer "B.Cu") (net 4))
 (segment (start 91.44 50.8) (end 75.692 50.8) (width 2.4) (layer "B.Cu") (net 4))
 (segment (start 52.07 60.96) (end 54.356 63.246) (width 1.6) (layer "B.Cu") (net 4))
 (segment (start 35.052 56.134) (end 35.052 62.992) (width 1.6) (layer "B.Cu") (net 4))
 (segment (start 35.052 53.594) (end 35.052 56.134) (width 1.6) (layer "B.Cu") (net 4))
 (segment (start 54.356 63.246) (end 62.738 63.246) (width 1.6) (layer "B.Cu") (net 4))
 (segment (start 62.738 63.246) (end 62.992 63.5) (width 1.6) (layer "B.Cu") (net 4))
 (segment (start 50.8 60.96) (end 52.07 60.96) (width 1.6) (layer "B.Cu") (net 4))
 (segment (start 35.052 62.992) (end 35.052 65.532) (width 1.6) (layer "B.Cu") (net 4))
 (segment (start 40.132 62.992) (end 44.196 62.992) (width 1.6) (layer "B.Cu") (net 5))
 (segment (start 44.704 63.5) (end 46.99 63.5) (width 1.6) (layer "B.Cu") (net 5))
 (segment (start 44.196 62.992) (end 44.704 63.5) (width 1.6) (layer "B.Cu") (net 5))
 (segment (start 50.8 63.5) (end 46.99 63.5) (width 1.6) (layer "B.Cu") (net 5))
 (segment (start 46.99 66.04) (end 50.8 66.04) (width 1.6) (layer "B.Cu") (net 6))
 (segment (start 40.132 65.532) (end 42.164 65.532) (width 1.6) (layer "B.Cu") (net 6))
 (segment (start 42.672 66.04) (end 46.99 66.04) (width 1.6) (layer "B.Cu") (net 6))
 (segment (start 42.164 65.532) (end 42.672 66.04) (width 1.6) (layer "B.Cu") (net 6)))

